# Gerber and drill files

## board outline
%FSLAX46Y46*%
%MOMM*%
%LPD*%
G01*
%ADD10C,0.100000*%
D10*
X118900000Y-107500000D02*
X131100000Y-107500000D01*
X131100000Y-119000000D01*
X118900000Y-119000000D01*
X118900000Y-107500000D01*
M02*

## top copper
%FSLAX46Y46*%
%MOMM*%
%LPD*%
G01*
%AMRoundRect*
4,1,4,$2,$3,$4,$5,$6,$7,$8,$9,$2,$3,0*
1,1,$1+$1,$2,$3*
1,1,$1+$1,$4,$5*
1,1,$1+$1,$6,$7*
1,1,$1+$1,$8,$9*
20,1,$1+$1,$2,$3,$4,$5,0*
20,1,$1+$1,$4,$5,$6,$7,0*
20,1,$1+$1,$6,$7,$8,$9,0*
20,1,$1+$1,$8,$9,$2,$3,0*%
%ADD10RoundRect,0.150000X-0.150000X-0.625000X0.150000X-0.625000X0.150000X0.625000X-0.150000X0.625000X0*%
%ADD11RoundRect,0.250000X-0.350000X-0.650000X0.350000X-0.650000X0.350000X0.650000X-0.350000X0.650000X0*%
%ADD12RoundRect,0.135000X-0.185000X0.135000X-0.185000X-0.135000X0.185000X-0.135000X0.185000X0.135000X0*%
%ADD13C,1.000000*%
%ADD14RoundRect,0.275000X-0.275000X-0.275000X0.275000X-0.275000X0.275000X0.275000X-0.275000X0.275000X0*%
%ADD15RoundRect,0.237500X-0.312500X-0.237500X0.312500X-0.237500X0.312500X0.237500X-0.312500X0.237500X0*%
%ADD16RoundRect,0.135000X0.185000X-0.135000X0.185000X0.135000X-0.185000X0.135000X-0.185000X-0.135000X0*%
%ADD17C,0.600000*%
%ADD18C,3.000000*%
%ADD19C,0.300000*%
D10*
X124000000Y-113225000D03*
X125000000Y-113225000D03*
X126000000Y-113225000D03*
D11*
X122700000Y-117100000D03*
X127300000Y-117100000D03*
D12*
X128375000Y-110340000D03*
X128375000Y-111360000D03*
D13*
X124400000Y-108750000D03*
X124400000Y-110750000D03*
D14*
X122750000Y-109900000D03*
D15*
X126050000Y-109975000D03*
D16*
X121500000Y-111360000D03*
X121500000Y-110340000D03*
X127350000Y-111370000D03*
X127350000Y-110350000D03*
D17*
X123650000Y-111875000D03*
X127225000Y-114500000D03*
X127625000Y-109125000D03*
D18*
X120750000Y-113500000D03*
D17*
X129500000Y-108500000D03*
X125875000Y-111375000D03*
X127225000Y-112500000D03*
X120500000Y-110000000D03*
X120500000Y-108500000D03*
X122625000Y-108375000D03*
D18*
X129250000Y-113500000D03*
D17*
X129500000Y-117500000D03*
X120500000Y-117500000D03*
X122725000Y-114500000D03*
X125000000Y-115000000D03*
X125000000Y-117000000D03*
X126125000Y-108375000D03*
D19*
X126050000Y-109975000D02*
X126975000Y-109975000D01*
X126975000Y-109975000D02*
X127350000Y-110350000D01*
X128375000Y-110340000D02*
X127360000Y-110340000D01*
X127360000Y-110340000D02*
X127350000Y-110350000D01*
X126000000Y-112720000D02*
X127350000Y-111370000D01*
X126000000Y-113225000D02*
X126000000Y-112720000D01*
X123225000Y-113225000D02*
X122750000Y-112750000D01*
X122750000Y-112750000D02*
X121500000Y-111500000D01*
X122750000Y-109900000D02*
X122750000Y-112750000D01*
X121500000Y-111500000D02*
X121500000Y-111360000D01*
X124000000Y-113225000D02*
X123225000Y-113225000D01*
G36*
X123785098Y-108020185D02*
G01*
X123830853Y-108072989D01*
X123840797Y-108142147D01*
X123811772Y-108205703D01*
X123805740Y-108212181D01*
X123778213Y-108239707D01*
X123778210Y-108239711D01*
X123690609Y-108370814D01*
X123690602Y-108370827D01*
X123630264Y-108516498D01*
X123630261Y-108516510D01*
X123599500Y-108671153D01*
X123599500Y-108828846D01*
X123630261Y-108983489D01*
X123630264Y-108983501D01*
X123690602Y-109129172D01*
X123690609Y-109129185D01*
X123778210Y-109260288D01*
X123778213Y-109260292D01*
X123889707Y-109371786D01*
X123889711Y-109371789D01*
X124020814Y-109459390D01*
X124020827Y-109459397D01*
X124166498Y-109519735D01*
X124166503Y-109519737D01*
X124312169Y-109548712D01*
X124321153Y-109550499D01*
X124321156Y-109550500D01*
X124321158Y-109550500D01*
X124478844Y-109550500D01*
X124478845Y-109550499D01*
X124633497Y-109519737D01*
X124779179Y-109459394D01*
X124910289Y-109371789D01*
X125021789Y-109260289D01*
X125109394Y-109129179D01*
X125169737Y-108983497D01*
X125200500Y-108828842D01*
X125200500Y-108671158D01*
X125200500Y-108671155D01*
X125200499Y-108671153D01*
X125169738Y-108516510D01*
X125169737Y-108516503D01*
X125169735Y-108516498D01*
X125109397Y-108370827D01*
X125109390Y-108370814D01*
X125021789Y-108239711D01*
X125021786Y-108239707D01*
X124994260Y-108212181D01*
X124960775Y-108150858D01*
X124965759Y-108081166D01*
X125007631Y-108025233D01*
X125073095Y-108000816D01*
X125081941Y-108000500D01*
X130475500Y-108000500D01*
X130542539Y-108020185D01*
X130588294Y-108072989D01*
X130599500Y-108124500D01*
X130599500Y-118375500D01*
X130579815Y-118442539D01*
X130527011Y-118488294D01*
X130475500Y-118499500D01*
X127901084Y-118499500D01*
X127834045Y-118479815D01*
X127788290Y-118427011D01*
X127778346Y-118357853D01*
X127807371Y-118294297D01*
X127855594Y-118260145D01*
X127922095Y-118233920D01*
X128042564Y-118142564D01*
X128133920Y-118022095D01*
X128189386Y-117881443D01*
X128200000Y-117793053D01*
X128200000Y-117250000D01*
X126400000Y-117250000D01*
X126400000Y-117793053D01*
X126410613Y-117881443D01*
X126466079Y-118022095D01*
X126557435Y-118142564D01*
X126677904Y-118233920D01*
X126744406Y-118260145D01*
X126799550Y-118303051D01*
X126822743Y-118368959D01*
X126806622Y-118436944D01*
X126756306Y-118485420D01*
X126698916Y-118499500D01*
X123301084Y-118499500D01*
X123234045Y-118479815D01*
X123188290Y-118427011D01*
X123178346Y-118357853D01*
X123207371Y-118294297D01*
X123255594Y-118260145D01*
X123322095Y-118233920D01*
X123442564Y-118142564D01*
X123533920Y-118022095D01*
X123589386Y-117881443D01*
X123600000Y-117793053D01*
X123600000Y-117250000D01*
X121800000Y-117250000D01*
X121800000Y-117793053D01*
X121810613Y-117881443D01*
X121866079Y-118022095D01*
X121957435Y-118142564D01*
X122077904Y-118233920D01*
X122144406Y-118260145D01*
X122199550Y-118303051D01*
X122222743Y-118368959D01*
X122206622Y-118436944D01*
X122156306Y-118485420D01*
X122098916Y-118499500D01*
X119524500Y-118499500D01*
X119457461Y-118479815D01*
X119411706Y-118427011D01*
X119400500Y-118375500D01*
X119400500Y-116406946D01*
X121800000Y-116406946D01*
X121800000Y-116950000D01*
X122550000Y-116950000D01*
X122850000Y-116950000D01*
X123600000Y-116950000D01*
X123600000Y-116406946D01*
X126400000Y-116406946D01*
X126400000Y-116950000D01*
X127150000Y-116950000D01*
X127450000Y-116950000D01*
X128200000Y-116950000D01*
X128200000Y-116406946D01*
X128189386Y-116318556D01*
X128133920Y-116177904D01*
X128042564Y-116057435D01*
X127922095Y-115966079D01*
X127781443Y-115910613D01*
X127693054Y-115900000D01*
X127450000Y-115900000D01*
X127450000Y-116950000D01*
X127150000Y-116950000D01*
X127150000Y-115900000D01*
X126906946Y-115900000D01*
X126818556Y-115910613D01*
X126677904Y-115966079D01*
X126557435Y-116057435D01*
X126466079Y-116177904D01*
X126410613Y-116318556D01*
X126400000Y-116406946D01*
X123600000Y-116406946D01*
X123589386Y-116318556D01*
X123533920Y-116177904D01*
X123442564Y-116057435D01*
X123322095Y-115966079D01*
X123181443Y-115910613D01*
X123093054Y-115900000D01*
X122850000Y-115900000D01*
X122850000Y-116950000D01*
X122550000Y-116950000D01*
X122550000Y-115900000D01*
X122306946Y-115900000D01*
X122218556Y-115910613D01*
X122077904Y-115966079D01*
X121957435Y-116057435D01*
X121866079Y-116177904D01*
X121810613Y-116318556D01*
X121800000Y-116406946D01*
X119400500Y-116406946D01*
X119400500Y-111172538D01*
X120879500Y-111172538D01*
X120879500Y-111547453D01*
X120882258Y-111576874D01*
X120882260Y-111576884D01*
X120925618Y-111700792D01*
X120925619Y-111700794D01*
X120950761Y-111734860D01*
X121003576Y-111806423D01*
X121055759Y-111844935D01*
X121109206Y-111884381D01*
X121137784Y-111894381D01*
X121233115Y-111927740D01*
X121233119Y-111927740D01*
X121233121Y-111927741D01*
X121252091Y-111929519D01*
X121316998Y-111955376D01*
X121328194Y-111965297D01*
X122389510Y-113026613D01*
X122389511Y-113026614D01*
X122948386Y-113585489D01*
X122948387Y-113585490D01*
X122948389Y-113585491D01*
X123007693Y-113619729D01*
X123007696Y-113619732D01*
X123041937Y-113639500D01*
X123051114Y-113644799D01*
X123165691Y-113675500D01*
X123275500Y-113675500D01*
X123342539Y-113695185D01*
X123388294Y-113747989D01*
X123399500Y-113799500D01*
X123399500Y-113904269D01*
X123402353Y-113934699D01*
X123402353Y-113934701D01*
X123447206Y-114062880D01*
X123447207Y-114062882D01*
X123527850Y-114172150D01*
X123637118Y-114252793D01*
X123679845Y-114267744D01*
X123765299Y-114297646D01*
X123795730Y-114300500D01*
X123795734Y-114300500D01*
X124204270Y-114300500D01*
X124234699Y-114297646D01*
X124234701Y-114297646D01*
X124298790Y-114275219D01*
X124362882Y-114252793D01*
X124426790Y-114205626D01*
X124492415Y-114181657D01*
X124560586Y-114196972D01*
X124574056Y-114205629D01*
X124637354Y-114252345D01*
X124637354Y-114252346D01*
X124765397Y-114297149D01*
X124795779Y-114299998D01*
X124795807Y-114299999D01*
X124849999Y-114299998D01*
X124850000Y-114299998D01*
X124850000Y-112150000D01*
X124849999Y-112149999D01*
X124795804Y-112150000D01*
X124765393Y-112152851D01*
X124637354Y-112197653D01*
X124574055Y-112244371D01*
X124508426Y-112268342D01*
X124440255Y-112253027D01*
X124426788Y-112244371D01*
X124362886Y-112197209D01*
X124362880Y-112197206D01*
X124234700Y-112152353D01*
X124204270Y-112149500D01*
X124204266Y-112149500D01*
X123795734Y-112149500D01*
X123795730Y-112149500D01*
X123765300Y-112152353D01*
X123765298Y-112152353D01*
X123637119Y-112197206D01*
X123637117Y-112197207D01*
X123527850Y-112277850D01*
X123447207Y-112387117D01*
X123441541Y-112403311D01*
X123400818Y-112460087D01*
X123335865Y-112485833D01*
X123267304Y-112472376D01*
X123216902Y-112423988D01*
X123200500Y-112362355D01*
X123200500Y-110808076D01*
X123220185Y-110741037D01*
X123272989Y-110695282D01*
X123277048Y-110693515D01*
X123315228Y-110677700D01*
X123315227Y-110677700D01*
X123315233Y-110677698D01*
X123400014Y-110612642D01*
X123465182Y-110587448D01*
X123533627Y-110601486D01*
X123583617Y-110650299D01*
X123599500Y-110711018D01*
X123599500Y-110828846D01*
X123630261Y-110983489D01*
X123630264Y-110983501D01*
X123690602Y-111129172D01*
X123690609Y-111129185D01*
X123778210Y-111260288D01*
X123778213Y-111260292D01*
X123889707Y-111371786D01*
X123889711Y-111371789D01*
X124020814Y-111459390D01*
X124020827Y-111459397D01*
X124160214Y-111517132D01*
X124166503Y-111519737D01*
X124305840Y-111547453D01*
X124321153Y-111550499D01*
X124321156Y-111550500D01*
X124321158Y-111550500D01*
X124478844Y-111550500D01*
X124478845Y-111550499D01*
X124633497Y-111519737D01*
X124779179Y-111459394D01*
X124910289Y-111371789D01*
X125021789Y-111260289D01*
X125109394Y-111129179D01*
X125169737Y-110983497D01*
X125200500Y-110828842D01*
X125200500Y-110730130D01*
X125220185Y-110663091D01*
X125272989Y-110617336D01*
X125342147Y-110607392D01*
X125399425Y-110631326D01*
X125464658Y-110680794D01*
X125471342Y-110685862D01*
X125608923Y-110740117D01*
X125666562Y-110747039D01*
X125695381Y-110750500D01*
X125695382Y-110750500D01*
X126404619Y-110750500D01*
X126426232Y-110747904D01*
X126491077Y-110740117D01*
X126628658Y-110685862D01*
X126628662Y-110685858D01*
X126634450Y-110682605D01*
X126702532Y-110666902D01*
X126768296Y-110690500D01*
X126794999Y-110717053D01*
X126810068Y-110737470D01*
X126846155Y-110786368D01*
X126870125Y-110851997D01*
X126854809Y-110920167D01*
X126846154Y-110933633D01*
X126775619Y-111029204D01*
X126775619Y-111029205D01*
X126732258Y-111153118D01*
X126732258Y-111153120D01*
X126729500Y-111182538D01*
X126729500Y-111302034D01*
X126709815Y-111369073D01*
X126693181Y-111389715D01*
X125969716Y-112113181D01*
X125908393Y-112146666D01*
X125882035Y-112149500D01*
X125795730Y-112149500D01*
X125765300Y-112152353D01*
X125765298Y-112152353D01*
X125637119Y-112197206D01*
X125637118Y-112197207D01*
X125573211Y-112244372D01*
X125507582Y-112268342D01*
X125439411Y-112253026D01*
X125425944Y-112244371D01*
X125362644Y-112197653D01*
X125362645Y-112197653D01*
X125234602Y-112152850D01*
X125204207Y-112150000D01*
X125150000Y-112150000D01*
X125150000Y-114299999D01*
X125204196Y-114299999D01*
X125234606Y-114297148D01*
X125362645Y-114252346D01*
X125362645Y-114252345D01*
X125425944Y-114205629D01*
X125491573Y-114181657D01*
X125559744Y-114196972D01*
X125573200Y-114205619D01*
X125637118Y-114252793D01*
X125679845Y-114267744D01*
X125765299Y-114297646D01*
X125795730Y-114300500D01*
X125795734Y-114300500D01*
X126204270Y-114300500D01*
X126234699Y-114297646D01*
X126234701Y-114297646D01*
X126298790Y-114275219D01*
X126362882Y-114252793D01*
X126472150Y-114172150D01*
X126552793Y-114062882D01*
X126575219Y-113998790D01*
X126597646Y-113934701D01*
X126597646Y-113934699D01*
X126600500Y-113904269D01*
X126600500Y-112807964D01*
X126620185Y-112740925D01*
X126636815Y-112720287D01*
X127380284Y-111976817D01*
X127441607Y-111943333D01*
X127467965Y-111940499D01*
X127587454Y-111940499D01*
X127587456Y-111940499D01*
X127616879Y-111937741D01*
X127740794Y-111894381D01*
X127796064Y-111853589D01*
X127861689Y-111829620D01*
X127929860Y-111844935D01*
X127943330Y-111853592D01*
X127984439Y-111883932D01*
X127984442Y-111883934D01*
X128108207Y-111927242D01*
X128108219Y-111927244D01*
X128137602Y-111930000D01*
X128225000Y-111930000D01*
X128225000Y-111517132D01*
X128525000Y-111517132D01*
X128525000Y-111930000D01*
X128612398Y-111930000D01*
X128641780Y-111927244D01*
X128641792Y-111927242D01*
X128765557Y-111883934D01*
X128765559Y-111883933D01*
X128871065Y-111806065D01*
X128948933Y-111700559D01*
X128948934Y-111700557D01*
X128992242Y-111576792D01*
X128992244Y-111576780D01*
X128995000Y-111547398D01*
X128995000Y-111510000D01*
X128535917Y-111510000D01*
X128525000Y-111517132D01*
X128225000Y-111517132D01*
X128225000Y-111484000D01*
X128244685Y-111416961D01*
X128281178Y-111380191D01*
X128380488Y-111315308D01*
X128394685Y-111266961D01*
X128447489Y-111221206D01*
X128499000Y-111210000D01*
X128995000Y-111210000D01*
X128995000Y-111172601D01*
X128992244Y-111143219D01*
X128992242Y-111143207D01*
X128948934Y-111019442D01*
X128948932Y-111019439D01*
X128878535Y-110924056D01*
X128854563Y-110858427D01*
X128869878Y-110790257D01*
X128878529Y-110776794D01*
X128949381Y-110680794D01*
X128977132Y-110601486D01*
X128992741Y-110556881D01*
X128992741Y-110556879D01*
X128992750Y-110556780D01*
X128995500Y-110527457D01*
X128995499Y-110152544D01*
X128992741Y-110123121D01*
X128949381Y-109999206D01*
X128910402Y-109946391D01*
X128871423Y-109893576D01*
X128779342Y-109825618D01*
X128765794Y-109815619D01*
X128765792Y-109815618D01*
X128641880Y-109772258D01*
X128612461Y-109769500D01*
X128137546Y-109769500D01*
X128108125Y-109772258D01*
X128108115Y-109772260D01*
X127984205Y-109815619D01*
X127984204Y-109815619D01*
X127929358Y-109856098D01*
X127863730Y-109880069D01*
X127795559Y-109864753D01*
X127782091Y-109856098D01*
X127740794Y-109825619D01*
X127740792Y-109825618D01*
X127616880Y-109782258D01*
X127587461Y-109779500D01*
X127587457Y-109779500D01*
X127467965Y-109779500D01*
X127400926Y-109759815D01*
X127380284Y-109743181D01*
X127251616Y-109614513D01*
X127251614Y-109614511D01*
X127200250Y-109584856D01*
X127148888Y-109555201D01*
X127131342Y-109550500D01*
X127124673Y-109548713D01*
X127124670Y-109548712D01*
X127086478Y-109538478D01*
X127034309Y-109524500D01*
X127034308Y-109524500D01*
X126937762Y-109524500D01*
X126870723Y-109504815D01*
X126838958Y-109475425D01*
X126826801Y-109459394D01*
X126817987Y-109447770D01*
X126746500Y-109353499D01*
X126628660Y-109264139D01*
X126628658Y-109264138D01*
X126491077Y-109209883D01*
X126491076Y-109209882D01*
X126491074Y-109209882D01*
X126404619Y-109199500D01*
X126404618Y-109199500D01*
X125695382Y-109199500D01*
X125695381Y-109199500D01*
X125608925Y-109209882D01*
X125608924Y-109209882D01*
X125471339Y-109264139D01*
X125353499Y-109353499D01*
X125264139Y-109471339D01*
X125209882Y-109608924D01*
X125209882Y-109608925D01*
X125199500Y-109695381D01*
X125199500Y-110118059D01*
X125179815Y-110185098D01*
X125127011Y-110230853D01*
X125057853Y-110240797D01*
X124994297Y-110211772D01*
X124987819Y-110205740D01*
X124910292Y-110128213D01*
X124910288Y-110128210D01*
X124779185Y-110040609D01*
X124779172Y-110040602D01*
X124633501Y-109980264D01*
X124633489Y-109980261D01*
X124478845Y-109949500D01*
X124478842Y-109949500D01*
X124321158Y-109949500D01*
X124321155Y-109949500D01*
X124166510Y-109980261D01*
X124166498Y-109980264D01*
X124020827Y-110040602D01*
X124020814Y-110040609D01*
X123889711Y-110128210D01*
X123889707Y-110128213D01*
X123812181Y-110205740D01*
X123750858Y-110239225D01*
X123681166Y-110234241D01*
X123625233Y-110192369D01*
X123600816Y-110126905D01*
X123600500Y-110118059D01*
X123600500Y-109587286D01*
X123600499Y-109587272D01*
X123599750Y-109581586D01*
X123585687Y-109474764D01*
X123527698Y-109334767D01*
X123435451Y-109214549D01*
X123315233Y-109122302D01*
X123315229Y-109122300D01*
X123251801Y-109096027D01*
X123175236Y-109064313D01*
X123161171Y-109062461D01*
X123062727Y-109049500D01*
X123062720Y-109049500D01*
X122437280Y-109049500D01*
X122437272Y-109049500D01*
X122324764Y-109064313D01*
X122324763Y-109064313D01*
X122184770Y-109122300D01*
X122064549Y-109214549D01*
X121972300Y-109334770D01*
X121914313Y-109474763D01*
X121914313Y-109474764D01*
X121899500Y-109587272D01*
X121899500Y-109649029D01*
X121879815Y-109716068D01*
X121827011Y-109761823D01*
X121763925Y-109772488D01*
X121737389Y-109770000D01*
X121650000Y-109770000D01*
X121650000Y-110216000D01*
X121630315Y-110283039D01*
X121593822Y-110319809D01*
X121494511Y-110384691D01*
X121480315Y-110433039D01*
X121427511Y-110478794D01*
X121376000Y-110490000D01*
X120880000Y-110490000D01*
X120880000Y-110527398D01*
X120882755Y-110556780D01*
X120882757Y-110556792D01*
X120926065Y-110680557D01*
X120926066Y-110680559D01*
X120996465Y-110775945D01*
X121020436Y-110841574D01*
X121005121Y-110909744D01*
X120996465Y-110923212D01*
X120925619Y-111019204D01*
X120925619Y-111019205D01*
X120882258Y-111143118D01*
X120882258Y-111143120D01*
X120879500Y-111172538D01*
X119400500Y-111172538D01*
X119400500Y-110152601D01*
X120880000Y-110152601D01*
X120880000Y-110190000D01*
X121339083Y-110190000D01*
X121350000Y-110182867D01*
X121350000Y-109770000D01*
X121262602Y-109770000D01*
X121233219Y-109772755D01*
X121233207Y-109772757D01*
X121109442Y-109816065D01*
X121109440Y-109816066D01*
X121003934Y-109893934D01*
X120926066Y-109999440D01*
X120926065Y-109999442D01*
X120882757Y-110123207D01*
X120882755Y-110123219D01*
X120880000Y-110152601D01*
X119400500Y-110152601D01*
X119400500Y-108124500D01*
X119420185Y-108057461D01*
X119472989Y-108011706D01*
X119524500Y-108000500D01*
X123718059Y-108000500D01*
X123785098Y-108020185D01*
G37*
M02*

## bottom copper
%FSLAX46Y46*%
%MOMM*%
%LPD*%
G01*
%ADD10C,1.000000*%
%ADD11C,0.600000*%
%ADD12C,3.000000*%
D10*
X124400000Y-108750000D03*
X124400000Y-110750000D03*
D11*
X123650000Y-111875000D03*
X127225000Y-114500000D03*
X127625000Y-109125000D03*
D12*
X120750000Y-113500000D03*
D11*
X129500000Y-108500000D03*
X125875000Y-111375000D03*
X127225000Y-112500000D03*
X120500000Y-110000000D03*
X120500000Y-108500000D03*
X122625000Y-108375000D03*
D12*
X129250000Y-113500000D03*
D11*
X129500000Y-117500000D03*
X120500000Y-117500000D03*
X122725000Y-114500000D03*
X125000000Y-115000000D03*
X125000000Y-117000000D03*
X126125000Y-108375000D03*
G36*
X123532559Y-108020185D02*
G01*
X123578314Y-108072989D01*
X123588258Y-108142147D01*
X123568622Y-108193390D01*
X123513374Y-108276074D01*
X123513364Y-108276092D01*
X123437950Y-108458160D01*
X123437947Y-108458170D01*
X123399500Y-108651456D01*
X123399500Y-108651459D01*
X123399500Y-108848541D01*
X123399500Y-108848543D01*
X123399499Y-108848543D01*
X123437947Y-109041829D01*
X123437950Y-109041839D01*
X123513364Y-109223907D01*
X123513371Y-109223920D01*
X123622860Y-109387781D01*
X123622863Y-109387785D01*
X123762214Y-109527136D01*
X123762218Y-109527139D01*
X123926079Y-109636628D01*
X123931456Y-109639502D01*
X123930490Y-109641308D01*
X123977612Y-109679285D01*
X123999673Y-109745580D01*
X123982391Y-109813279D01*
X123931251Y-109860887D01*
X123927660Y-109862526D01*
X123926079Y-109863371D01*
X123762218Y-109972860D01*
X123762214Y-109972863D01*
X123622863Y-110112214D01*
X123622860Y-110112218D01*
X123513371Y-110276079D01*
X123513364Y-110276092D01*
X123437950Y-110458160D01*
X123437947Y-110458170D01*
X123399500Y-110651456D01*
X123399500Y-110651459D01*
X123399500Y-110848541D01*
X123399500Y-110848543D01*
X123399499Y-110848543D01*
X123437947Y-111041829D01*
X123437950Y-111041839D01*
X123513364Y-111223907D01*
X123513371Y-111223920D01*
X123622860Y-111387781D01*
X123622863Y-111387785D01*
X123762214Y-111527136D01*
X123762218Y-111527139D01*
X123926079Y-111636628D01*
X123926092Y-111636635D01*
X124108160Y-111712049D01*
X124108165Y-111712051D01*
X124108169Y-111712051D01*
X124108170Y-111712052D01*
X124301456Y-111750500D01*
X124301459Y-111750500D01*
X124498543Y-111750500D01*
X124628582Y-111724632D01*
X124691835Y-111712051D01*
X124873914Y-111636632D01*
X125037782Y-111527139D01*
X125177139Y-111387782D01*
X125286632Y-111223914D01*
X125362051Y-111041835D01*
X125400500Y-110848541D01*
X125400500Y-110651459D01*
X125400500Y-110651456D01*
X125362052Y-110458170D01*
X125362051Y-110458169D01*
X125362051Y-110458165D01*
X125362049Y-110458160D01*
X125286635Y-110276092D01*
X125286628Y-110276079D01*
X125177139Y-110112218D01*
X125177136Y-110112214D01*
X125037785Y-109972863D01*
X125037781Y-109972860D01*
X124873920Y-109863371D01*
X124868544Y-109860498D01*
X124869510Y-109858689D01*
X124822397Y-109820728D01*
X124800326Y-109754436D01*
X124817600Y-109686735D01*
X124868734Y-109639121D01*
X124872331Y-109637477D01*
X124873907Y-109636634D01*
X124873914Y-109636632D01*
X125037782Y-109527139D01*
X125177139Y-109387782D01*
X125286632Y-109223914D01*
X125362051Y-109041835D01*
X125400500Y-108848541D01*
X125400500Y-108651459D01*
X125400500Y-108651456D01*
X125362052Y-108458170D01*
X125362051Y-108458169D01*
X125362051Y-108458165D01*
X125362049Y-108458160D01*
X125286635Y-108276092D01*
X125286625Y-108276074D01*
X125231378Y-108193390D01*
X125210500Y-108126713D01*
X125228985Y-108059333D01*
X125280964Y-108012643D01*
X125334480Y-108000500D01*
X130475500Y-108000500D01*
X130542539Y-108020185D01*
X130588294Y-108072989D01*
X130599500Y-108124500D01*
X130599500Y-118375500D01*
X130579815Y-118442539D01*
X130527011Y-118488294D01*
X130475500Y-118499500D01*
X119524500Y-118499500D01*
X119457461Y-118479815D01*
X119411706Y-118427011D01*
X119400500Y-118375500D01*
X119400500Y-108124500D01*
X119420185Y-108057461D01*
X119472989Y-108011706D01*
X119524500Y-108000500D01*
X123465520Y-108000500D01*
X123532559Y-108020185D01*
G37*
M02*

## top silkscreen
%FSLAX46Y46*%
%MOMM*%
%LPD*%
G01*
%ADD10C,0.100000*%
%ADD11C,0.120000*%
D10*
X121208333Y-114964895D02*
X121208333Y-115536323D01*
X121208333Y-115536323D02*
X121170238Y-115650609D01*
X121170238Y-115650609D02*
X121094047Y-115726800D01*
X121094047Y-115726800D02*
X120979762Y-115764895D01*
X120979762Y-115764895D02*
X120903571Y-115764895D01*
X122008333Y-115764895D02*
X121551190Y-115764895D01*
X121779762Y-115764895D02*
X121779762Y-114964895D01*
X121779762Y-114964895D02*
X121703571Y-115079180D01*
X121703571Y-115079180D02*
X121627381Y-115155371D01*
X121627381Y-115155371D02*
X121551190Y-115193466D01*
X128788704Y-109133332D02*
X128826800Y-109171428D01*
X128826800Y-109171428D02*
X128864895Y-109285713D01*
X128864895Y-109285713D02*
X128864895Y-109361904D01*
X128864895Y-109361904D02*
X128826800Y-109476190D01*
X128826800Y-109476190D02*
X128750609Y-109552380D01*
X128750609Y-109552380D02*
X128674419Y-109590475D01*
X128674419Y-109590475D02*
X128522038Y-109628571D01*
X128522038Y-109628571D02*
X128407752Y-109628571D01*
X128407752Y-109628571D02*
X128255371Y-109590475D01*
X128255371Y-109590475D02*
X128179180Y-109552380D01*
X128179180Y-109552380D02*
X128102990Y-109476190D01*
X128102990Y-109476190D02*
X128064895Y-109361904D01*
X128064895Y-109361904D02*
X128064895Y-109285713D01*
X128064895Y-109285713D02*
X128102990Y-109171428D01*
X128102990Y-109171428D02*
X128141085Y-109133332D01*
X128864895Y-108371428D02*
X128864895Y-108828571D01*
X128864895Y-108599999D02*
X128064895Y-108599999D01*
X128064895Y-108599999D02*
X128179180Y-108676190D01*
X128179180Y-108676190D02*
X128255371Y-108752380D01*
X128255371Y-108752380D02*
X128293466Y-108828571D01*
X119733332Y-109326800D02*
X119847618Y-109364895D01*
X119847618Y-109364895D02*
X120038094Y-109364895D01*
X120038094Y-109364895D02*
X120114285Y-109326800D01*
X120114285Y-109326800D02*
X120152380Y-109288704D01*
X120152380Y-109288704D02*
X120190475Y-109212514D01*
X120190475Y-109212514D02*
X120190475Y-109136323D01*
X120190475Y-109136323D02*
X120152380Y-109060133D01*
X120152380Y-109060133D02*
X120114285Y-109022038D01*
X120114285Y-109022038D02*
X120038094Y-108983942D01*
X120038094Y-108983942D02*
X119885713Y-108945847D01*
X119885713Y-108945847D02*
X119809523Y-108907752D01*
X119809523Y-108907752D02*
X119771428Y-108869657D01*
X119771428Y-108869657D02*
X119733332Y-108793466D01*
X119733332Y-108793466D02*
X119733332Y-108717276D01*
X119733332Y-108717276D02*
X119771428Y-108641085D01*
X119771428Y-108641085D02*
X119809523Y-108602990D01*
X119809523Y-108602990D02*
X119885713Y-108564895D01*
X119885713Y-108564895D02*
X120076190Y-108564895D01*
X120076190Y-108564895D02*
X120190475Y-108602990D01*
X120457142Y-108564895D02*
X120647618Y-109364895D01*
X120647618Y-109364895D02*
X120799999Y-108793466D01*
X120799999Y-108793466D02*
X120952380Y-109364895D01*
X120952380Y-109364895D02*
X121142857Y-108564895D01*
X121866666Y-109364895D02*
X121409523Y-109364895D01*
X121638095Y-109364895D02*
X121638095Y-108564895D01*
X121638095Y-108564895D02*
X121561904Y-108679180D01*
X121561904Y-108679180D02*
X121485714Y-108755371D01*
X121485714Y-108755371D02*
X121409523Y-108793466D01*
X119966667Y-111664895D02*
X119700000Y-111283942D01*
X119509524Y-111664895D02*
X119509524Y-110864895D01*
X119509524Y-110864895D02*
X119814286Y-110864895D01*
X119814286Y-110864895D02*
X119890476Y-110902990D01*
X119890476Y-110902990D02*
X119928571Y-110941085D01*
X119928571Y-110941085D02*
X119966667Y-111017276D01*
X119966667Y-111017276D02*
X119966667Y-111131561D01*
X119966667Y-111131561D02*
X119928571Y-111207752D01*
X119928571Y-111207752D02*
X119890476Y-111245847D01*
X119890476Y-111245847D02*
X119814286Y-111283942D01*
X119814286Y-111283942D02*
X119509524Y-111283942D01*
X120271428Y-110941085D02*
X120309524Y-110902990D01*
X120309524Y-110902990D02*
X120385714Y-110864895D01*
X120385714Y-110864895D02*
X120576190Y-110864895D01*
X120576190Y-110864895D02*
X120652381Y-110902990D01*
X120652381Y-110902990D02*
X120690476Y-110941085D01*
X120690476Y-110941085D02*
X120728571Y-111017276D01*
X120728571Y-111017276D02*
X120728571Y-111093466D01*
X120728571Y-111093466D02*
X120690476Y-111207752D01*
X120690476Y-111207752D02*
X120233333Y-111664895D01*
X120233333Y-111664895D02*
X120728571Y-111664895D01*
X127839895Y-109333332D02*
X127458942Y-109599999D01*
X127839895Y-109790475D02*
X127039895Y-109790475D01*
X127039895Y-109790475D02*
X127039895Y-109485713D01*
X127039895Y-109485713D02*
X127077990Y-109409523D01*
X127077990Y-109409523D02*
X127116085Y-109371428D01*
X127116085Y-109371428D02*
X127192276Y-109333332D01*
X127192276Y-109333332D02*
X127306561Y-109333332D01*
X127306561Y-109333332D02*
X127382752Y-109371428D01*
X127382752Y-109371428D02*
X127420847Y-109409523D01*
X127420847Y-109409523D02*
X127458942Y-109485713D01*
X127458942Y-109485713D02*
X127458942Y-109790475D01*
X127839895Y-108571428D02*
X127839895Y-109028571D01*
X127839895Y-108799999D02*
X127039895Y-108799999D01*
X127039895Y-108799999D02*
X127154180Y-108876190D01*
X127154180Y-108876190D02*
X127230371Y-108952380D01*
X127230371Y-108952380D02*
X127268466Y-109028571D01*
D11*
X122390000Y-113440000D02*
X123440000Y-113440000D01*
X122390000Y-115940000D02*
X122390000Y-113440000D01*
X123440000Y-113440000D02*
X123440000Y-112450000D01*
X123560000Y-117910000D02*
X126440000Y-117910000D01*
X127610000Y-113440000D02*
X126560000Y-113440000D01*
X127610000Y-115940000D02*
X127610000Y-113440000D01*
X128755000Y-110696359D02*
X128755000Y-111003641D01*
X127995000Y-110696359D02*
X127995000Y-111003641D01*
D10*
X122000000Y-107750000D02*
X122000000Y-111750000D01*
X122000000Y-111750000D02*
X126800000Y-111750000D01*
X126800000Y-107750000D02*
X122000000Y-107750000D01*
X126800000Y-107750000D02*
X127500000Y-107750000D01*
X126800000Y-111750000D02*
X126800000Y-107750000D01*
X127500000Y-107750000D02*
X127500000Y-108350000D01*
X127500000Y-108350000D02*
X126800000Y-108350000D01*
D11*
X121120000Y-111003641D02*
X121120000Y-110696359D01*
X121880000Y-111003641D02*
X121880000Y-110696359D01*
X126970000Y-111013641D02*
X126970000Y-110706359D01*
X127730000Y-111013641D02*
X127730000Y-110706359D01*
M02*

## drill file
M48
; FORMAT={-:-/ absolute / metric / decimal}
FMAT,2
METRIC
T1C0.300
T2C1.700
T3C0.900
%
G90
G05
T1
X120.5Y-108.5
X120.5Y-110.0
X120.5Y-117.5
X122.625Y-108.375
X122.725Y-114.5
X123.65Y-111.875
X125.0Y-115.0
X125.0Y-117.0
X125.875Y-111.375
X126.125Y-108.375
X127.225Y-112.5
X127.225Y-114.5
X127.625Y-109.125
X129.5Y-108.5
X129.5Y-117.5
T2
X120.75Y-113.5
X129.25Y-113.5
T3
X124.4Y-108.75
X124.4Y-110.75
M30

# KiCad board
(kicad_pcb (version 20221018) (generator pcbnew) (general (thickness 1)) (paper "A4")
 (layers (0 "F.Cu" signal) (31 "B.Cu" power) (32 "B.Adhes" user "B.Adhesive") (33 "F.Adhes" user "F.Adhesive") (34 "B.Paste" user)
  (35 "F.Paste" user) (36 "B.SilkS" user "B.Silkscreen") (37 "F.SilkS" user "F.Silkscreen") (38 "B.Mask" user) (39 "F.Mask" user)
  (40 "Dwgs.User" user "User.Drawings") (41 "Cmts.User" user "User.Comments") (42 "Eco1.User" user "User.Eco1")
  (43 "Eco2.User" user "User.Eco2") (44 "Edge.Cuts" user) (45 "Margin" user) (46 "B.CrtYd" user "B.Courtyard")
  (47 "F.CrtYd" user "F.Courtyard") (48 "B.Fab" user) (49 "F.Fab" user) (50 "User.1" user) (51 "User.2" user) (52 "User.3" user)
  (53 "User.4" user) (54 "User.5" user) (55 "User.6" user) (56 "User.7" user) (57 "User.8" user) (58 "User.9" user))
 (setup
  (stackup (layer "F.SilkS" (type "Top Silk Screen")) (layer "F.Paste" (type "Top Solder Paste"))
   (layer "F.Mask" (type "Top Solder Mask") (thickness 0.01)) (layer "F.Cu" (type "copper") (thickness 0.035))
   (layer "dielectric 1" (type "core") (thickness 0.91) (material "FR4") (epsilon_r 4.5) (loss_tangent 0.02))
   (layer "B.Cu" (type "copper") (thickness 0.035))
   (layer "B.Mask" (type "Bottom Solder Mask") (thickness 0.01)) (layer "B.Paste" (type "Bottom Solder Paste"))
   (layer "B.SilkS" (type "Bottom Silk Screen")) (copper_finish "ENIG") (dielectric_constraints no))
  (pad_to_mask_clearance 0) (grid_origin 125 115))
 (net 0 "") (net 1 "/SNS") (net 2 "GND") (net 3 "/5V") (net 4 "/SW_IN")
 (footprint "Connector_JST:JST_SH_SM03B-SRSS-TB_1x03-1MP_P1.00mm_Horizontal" (layer "F.Cu") (at 125 115.225)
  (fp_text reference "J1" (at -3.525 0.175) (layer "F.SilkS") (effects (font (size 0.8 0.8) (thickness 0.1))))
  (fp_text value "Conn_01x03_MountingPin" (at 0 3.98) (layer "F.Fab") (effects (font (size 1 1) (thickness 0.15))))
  (fp_line (start -2.61 -1.785) (end -1.56 -1.785) (stroke (width 0.12) (type solid)) (layer "F.SilkS"))
  (fp_line (start -2.61 0.715) (end -2.61 -1.785) (stroke (width 0.12) (type solid)) (layer "F.SilkS"))
  (fp_line (start -1.56 -1.785) (end -1.56 -2.775) (stroke (width 0.12) (type solid)) (layer "F.SilkS"))
  (fp_line (start -1.44 2.685) (end 1.44 2.685) (stroke (width 0.12) (type solid)) (layer "F.SilkS"))
  (fp_line (start 2.61 -1.785) (end 1.56 -1.785) (stroke (width 0.12) (type solid)) (layer "F.SilkS"))
  (fp_line (start 2.61 0.715) (end 2.61 -1.785) (stroke (width 0.12) (type solid)) (layer "F.SilkS"))
  (pad "1" smd roundrect (at -1 -2) (size 0.6 1.55) (layers "F.Cu" "F.Paste" "F.Mask") (roundrect_rratio 0.25) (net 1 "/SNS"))
  (pad "2" smd roundrect (at 0 -2) (size 0.6 1.55) (layers "F.Cu" "F.Paste" "F.Mask") (roundrect_rratio 0.25) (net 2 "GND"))
  (pad "3" smd roundrect (at 1 -2) (size 0.6 1.55) (layers "F.Cu" "F.Paste" "F.Mask") (roundrect_rratio 0.25) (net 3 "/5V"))
  (pad "MP" smd roundrect (at -2.3 1.875) (size 1.2 1.8) (layers "F.Cu" "F.Paste" "F.Mask") (roundrect_rratio 0.2083333333) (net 2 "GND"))
  (pad "MP" smd roundrect (at 2.3 1.875) (size 1.2 1.8) (layers "F.Cu" "F.Paste" "F.Mask") (roundrect_rratio 0.2083333333) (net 2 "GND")))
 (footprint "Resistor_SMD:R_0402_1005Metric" (layer "F.Cu") (at 128.375 110.85 -90)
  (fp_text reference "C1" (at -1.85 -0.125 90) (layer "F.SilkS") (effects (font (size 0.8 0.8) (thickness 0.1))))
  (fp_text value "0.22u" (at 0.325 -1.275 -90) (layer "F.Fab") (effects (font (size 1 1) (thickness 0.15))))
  (fp_line (start -0.153641 -0.38) (end 0.153641 -0.38) (stroke (width 0.12) (type solid)) (layer "F.SilkS"))
  (fp_line (start -0.153641 0.38) (end 0.153641 0.38) (stroke (width 0.12) (type solid)) (layer "F.SilkS"))
  (pad "1" smd roundrect (at -0.51 0 270) (size 0.54 0.64) (layers "F.Cu" "F.Paste" "F.Mask") (roundrect_rratio 0.25) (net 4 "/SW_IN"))
  (pad "2" smd roundrect (at 0.51 0 270) (size 0.54 0.64) (layers "F.Cu" "F.Paste" "F.Mask") (roundrect_rratio 0.25) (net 2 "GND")))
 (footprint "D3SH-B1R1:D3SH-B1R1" (layer "F.Cu") (at 124.4 111.55)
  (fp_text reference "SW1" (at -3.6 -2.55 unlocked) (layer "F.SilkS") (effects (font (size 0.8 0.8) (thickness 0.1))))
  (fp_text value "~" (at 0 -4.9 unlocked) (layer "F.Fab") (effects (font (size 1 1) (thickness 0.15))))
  (fp_line (start -2.4 -3.8) (end -2.4 0.2) (stroke (width 0.1) (type default)) (layer "F.SilkS"))
  (fp_line (start -2.4 0.2) (end 2.4 0.2) (stroke (width 0.1) (type default)) (layer "F.SilkS"))
  (fp_line (start 2.4 -3.8) (end -2.4 -3.8) (stroke (width 0.1) (type default)) (layer "F.SilkS"))
  (fp_line (start 2.4 -3.8) (end 3.1 -3.8) (stroke (width 0.1) (type default)) (layer "F.SilkS"))
  (fp_line (start 2.4 0.2) (end 2.4 -3.8) (stroke (width 0.1) (type default)) (layer "F.SilkS"))
  (fp_line (start 3.1 -3.8) (end 3.1 -3.2) (stroke (width 0.1) (type default)) (layer "F.SilkS"))
  (fp_line (start 3.1 -3.2) (end 2.4 -3.2) (stroke (width 0.1) (type default)) (layer "F.SilkS"))
  (pad "" np_thru_hole circle (at 0 -2.8) (size 1 1) (drill 0.9) (layers "*.Cu" "*.Mask"))
  (pad "" np_thru_hole circle (at 0 -0.8) (size 1 1) (drill 0.9) (layers "*.Cu" "*.Mask"))
  (pad "1" smd roundrect (at -1.65 -1.65) (size 1.1 1.1) (layers "F.Cu" "F.Paste" "F.Mask") (roundrect_rratio 0.25) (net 1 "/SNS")
   (thermal_bridge_angle 45))
  (pad "2" smd roundrect (at 1.65 -1.575) (size 1.1 0.95) (layers "F.Cu" "F.Paste" "F.Mask") (roundrect_rratio 0.25) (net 4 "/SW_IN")
   (thermal_bridge_angle 45)))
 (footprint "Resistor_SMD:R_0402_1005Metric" (layer "F.Cu") (at 121.5 110.85 90)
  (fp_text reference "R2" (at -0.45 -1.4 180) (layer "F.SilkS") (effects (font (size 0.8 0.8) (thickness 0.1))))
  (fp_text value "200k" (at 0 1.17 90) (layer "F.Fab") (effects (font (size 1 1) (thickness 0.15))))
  (fp_line (start -0.153641 -0.38) (end 0.153641 -0.38) (stroke (width 0.12) (type solid)) (layer "F.SilkS"))
  (fp_line (start -0.153641 0.38) (end 0.153641 0.38) (stroke (width 0.12) (type solid)) (layer "F.SilkS"))
  (pad "1" smd roundrect (at -0.51 0 90) (size 0.54 0.64) (layers "F.Cu" "F.Paste" "F.Mask") (roundrect_rratio 0.25) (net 1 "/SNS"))
  (pad "2" smd roundrect (at 0.51 0 90) (size 0.54 0.64) (layers "F.Cu" "F.Paste" "F.Mask") (roundrect_rratio 0.25) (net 2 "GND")))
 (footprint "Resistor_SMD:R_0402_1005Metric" (layer "F.Cu") (at 127.35 110.86 90)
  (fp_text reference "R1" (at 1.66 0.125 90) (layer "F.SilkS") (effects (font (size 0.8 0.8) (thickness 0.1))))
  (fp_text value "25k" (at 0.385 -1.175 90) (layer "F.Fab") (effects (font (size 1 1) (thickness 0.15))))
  (fp_line (start -0.153641 -0.38) (end 0.153641 -0.38) (stroke (width 0.12) (type solid)) (layer "F.SilkS"))
  (fp_line (start -0.153641 0.38) (end 0.153641 0.38) (stroke (width 0.12) (type solid)) (layer "F.SilkS"))
  (pad "1" smd roundrect (at -0.51 0 90) (size 0.54 0.64) (layers "F.Cu" "F.Paste" "F.Mask") (roundrect_rratio 0.25) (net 3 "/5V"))
  (pad "2" smd roundrect (at 0.51 0 90) (size 0.54 0.64) (layers "F.Cu" "F.Paste" "F.Mask") (roundrect_rratio 0.25) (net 4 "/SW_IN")))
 (gr_rect (start 118.9 107.5) (end 131.1 119) (stroke (width 0.1) (type default)) (fill none) (layer "Edge.Cuts"))
 (via (at 123.65 111.875) (size 0.6) (drill 0.3) (layers "F.Cu" "B.Cu") (free) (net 2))
 (via (at 127.225 114.5) (size 0.6) (drill 0.3) (layers "F.Cu" "B.Cu") (free) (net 2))
 (via (at 127.625 109.125) (size 0.6) (drill 0.3) (layers "F.Cu" "B.Cu") (free) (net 2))
 (via (at 120.75 113.5) (size 3) (drill 1.7) (layers "F.Cu" "B.Cu") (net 2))
 (via (at 129.5 108.5) (size 0.6) (drill 0.3) (layers "F.Cu" "B.Cu") (free) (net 2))
 (via (at 125.875 111.375) (size 0.6) (drill 0.3) (layers "F.Cu" "B.Cu") (free) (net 2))
 (via (at 127.225 112.5) (size 0.6) (drill 0.3) (layers "F.Cu" "B.Cu") (free) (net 2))
 (via (at 120.5 110) (size 0.6) (drill 0.3) (layers "F.Cu" "B.Cu") (free) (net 2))
 (via (at 120.5 108.5) (size 0.6) (drill 0.3) (layers "F.Cu" "B.Cu") (free) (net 2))
 (via (at 122.625 108.375) (size 0.6) (drill 0.3) (layers "F.Cu" "B.Cu") (free) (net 2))
 (via (at 129.25 113.5) (size 3) (drill 1.7) (layers "F.Cu" "B.Cu") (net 2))
 (via (at 129.5 117.5) (size 0.6) (drill 0.3) (layers "F.Cu" "B.Cu") (free) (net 2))
 (via (at 120.5 117.5) (size 0.6) (drill 0.3) (layers "F.Cu" "B.Cu") (free) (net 2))
 (via (at 122.725 114.5) (size 0.6) (drill 0.3) (layers "F.Cu" "B.Cu") (free) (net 2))
 (via (at 125 115) (size 0.6) (drill 0.3) (layers "F.Cu" "B.Cu") (free) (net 2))
 (via (at 125 117) (size 0.6) (drill 0.3) (layers "F.Cu" "B.Cu") (free) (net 2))
 (via (at 126.125 108.375) (size 0.6) (drill 0.3) (layers "F.Cu" "B.Cu") (free) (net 2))
 (segment (start 126.05 109.975) (end 126.975 109.975) (width 0.3) (layer "F.Cu") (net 4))
 (segment (start 126.975 109.975) (end 127.35 110.35) (width 0.3) (layer "F.Cu") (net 4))
 (segment (start 128.375 110.34) (end 127.36 110.34) (width 0.3) (layer "F.Cu") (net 4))
 (segment (start 127.36 110.34) (end 127.35 110.35) (width 0.3) (layer "F.Cu") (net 4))
 (segment (start 126 112.72) (end 127.35 111.37) (width 0.3) (layer "F.Cu") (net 3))
 (segment (start 126 113.225) (end 126 112.72) (width 0.3) (layer "F.Cu") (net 3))
 (segment (start 123.225 113.225) (end 122.75 112.75) (width 0.3) (layer "F.Cu") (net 1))
 (segment (start 122.75 112.75) (end 121.5 111.5) (width 0.3) (layer "F.Cu") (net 1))
 (segment (start 122.75 109.9) (end 122.75 112.75) (width 0.3) (layer "F.Cu") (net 1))
 (segment (start 121.5 111.5) (end 121.5 111.36) (width 0.3) (layer "F.Cu") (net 1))
 (segment (start 124 113.225) (end 123.225 113.225) (width 0.3) (layer "F.Cu") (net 1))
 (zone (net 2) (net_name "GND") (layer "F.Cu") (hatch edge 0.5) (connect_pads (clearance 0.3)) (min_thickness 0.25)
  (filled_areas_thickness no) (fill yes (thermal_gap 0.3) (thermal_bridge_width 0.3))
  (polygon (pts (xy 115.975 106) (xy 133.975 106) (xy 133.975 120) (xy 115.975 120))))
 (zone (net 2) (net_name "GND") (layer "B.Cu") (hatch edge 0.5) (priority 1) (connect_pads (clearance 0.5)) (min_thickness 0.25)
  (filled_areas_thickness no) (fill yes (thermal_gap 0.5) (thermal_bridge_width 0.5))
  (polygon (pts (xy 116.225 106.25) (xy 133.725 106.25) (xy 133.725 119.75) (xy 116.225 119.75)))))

